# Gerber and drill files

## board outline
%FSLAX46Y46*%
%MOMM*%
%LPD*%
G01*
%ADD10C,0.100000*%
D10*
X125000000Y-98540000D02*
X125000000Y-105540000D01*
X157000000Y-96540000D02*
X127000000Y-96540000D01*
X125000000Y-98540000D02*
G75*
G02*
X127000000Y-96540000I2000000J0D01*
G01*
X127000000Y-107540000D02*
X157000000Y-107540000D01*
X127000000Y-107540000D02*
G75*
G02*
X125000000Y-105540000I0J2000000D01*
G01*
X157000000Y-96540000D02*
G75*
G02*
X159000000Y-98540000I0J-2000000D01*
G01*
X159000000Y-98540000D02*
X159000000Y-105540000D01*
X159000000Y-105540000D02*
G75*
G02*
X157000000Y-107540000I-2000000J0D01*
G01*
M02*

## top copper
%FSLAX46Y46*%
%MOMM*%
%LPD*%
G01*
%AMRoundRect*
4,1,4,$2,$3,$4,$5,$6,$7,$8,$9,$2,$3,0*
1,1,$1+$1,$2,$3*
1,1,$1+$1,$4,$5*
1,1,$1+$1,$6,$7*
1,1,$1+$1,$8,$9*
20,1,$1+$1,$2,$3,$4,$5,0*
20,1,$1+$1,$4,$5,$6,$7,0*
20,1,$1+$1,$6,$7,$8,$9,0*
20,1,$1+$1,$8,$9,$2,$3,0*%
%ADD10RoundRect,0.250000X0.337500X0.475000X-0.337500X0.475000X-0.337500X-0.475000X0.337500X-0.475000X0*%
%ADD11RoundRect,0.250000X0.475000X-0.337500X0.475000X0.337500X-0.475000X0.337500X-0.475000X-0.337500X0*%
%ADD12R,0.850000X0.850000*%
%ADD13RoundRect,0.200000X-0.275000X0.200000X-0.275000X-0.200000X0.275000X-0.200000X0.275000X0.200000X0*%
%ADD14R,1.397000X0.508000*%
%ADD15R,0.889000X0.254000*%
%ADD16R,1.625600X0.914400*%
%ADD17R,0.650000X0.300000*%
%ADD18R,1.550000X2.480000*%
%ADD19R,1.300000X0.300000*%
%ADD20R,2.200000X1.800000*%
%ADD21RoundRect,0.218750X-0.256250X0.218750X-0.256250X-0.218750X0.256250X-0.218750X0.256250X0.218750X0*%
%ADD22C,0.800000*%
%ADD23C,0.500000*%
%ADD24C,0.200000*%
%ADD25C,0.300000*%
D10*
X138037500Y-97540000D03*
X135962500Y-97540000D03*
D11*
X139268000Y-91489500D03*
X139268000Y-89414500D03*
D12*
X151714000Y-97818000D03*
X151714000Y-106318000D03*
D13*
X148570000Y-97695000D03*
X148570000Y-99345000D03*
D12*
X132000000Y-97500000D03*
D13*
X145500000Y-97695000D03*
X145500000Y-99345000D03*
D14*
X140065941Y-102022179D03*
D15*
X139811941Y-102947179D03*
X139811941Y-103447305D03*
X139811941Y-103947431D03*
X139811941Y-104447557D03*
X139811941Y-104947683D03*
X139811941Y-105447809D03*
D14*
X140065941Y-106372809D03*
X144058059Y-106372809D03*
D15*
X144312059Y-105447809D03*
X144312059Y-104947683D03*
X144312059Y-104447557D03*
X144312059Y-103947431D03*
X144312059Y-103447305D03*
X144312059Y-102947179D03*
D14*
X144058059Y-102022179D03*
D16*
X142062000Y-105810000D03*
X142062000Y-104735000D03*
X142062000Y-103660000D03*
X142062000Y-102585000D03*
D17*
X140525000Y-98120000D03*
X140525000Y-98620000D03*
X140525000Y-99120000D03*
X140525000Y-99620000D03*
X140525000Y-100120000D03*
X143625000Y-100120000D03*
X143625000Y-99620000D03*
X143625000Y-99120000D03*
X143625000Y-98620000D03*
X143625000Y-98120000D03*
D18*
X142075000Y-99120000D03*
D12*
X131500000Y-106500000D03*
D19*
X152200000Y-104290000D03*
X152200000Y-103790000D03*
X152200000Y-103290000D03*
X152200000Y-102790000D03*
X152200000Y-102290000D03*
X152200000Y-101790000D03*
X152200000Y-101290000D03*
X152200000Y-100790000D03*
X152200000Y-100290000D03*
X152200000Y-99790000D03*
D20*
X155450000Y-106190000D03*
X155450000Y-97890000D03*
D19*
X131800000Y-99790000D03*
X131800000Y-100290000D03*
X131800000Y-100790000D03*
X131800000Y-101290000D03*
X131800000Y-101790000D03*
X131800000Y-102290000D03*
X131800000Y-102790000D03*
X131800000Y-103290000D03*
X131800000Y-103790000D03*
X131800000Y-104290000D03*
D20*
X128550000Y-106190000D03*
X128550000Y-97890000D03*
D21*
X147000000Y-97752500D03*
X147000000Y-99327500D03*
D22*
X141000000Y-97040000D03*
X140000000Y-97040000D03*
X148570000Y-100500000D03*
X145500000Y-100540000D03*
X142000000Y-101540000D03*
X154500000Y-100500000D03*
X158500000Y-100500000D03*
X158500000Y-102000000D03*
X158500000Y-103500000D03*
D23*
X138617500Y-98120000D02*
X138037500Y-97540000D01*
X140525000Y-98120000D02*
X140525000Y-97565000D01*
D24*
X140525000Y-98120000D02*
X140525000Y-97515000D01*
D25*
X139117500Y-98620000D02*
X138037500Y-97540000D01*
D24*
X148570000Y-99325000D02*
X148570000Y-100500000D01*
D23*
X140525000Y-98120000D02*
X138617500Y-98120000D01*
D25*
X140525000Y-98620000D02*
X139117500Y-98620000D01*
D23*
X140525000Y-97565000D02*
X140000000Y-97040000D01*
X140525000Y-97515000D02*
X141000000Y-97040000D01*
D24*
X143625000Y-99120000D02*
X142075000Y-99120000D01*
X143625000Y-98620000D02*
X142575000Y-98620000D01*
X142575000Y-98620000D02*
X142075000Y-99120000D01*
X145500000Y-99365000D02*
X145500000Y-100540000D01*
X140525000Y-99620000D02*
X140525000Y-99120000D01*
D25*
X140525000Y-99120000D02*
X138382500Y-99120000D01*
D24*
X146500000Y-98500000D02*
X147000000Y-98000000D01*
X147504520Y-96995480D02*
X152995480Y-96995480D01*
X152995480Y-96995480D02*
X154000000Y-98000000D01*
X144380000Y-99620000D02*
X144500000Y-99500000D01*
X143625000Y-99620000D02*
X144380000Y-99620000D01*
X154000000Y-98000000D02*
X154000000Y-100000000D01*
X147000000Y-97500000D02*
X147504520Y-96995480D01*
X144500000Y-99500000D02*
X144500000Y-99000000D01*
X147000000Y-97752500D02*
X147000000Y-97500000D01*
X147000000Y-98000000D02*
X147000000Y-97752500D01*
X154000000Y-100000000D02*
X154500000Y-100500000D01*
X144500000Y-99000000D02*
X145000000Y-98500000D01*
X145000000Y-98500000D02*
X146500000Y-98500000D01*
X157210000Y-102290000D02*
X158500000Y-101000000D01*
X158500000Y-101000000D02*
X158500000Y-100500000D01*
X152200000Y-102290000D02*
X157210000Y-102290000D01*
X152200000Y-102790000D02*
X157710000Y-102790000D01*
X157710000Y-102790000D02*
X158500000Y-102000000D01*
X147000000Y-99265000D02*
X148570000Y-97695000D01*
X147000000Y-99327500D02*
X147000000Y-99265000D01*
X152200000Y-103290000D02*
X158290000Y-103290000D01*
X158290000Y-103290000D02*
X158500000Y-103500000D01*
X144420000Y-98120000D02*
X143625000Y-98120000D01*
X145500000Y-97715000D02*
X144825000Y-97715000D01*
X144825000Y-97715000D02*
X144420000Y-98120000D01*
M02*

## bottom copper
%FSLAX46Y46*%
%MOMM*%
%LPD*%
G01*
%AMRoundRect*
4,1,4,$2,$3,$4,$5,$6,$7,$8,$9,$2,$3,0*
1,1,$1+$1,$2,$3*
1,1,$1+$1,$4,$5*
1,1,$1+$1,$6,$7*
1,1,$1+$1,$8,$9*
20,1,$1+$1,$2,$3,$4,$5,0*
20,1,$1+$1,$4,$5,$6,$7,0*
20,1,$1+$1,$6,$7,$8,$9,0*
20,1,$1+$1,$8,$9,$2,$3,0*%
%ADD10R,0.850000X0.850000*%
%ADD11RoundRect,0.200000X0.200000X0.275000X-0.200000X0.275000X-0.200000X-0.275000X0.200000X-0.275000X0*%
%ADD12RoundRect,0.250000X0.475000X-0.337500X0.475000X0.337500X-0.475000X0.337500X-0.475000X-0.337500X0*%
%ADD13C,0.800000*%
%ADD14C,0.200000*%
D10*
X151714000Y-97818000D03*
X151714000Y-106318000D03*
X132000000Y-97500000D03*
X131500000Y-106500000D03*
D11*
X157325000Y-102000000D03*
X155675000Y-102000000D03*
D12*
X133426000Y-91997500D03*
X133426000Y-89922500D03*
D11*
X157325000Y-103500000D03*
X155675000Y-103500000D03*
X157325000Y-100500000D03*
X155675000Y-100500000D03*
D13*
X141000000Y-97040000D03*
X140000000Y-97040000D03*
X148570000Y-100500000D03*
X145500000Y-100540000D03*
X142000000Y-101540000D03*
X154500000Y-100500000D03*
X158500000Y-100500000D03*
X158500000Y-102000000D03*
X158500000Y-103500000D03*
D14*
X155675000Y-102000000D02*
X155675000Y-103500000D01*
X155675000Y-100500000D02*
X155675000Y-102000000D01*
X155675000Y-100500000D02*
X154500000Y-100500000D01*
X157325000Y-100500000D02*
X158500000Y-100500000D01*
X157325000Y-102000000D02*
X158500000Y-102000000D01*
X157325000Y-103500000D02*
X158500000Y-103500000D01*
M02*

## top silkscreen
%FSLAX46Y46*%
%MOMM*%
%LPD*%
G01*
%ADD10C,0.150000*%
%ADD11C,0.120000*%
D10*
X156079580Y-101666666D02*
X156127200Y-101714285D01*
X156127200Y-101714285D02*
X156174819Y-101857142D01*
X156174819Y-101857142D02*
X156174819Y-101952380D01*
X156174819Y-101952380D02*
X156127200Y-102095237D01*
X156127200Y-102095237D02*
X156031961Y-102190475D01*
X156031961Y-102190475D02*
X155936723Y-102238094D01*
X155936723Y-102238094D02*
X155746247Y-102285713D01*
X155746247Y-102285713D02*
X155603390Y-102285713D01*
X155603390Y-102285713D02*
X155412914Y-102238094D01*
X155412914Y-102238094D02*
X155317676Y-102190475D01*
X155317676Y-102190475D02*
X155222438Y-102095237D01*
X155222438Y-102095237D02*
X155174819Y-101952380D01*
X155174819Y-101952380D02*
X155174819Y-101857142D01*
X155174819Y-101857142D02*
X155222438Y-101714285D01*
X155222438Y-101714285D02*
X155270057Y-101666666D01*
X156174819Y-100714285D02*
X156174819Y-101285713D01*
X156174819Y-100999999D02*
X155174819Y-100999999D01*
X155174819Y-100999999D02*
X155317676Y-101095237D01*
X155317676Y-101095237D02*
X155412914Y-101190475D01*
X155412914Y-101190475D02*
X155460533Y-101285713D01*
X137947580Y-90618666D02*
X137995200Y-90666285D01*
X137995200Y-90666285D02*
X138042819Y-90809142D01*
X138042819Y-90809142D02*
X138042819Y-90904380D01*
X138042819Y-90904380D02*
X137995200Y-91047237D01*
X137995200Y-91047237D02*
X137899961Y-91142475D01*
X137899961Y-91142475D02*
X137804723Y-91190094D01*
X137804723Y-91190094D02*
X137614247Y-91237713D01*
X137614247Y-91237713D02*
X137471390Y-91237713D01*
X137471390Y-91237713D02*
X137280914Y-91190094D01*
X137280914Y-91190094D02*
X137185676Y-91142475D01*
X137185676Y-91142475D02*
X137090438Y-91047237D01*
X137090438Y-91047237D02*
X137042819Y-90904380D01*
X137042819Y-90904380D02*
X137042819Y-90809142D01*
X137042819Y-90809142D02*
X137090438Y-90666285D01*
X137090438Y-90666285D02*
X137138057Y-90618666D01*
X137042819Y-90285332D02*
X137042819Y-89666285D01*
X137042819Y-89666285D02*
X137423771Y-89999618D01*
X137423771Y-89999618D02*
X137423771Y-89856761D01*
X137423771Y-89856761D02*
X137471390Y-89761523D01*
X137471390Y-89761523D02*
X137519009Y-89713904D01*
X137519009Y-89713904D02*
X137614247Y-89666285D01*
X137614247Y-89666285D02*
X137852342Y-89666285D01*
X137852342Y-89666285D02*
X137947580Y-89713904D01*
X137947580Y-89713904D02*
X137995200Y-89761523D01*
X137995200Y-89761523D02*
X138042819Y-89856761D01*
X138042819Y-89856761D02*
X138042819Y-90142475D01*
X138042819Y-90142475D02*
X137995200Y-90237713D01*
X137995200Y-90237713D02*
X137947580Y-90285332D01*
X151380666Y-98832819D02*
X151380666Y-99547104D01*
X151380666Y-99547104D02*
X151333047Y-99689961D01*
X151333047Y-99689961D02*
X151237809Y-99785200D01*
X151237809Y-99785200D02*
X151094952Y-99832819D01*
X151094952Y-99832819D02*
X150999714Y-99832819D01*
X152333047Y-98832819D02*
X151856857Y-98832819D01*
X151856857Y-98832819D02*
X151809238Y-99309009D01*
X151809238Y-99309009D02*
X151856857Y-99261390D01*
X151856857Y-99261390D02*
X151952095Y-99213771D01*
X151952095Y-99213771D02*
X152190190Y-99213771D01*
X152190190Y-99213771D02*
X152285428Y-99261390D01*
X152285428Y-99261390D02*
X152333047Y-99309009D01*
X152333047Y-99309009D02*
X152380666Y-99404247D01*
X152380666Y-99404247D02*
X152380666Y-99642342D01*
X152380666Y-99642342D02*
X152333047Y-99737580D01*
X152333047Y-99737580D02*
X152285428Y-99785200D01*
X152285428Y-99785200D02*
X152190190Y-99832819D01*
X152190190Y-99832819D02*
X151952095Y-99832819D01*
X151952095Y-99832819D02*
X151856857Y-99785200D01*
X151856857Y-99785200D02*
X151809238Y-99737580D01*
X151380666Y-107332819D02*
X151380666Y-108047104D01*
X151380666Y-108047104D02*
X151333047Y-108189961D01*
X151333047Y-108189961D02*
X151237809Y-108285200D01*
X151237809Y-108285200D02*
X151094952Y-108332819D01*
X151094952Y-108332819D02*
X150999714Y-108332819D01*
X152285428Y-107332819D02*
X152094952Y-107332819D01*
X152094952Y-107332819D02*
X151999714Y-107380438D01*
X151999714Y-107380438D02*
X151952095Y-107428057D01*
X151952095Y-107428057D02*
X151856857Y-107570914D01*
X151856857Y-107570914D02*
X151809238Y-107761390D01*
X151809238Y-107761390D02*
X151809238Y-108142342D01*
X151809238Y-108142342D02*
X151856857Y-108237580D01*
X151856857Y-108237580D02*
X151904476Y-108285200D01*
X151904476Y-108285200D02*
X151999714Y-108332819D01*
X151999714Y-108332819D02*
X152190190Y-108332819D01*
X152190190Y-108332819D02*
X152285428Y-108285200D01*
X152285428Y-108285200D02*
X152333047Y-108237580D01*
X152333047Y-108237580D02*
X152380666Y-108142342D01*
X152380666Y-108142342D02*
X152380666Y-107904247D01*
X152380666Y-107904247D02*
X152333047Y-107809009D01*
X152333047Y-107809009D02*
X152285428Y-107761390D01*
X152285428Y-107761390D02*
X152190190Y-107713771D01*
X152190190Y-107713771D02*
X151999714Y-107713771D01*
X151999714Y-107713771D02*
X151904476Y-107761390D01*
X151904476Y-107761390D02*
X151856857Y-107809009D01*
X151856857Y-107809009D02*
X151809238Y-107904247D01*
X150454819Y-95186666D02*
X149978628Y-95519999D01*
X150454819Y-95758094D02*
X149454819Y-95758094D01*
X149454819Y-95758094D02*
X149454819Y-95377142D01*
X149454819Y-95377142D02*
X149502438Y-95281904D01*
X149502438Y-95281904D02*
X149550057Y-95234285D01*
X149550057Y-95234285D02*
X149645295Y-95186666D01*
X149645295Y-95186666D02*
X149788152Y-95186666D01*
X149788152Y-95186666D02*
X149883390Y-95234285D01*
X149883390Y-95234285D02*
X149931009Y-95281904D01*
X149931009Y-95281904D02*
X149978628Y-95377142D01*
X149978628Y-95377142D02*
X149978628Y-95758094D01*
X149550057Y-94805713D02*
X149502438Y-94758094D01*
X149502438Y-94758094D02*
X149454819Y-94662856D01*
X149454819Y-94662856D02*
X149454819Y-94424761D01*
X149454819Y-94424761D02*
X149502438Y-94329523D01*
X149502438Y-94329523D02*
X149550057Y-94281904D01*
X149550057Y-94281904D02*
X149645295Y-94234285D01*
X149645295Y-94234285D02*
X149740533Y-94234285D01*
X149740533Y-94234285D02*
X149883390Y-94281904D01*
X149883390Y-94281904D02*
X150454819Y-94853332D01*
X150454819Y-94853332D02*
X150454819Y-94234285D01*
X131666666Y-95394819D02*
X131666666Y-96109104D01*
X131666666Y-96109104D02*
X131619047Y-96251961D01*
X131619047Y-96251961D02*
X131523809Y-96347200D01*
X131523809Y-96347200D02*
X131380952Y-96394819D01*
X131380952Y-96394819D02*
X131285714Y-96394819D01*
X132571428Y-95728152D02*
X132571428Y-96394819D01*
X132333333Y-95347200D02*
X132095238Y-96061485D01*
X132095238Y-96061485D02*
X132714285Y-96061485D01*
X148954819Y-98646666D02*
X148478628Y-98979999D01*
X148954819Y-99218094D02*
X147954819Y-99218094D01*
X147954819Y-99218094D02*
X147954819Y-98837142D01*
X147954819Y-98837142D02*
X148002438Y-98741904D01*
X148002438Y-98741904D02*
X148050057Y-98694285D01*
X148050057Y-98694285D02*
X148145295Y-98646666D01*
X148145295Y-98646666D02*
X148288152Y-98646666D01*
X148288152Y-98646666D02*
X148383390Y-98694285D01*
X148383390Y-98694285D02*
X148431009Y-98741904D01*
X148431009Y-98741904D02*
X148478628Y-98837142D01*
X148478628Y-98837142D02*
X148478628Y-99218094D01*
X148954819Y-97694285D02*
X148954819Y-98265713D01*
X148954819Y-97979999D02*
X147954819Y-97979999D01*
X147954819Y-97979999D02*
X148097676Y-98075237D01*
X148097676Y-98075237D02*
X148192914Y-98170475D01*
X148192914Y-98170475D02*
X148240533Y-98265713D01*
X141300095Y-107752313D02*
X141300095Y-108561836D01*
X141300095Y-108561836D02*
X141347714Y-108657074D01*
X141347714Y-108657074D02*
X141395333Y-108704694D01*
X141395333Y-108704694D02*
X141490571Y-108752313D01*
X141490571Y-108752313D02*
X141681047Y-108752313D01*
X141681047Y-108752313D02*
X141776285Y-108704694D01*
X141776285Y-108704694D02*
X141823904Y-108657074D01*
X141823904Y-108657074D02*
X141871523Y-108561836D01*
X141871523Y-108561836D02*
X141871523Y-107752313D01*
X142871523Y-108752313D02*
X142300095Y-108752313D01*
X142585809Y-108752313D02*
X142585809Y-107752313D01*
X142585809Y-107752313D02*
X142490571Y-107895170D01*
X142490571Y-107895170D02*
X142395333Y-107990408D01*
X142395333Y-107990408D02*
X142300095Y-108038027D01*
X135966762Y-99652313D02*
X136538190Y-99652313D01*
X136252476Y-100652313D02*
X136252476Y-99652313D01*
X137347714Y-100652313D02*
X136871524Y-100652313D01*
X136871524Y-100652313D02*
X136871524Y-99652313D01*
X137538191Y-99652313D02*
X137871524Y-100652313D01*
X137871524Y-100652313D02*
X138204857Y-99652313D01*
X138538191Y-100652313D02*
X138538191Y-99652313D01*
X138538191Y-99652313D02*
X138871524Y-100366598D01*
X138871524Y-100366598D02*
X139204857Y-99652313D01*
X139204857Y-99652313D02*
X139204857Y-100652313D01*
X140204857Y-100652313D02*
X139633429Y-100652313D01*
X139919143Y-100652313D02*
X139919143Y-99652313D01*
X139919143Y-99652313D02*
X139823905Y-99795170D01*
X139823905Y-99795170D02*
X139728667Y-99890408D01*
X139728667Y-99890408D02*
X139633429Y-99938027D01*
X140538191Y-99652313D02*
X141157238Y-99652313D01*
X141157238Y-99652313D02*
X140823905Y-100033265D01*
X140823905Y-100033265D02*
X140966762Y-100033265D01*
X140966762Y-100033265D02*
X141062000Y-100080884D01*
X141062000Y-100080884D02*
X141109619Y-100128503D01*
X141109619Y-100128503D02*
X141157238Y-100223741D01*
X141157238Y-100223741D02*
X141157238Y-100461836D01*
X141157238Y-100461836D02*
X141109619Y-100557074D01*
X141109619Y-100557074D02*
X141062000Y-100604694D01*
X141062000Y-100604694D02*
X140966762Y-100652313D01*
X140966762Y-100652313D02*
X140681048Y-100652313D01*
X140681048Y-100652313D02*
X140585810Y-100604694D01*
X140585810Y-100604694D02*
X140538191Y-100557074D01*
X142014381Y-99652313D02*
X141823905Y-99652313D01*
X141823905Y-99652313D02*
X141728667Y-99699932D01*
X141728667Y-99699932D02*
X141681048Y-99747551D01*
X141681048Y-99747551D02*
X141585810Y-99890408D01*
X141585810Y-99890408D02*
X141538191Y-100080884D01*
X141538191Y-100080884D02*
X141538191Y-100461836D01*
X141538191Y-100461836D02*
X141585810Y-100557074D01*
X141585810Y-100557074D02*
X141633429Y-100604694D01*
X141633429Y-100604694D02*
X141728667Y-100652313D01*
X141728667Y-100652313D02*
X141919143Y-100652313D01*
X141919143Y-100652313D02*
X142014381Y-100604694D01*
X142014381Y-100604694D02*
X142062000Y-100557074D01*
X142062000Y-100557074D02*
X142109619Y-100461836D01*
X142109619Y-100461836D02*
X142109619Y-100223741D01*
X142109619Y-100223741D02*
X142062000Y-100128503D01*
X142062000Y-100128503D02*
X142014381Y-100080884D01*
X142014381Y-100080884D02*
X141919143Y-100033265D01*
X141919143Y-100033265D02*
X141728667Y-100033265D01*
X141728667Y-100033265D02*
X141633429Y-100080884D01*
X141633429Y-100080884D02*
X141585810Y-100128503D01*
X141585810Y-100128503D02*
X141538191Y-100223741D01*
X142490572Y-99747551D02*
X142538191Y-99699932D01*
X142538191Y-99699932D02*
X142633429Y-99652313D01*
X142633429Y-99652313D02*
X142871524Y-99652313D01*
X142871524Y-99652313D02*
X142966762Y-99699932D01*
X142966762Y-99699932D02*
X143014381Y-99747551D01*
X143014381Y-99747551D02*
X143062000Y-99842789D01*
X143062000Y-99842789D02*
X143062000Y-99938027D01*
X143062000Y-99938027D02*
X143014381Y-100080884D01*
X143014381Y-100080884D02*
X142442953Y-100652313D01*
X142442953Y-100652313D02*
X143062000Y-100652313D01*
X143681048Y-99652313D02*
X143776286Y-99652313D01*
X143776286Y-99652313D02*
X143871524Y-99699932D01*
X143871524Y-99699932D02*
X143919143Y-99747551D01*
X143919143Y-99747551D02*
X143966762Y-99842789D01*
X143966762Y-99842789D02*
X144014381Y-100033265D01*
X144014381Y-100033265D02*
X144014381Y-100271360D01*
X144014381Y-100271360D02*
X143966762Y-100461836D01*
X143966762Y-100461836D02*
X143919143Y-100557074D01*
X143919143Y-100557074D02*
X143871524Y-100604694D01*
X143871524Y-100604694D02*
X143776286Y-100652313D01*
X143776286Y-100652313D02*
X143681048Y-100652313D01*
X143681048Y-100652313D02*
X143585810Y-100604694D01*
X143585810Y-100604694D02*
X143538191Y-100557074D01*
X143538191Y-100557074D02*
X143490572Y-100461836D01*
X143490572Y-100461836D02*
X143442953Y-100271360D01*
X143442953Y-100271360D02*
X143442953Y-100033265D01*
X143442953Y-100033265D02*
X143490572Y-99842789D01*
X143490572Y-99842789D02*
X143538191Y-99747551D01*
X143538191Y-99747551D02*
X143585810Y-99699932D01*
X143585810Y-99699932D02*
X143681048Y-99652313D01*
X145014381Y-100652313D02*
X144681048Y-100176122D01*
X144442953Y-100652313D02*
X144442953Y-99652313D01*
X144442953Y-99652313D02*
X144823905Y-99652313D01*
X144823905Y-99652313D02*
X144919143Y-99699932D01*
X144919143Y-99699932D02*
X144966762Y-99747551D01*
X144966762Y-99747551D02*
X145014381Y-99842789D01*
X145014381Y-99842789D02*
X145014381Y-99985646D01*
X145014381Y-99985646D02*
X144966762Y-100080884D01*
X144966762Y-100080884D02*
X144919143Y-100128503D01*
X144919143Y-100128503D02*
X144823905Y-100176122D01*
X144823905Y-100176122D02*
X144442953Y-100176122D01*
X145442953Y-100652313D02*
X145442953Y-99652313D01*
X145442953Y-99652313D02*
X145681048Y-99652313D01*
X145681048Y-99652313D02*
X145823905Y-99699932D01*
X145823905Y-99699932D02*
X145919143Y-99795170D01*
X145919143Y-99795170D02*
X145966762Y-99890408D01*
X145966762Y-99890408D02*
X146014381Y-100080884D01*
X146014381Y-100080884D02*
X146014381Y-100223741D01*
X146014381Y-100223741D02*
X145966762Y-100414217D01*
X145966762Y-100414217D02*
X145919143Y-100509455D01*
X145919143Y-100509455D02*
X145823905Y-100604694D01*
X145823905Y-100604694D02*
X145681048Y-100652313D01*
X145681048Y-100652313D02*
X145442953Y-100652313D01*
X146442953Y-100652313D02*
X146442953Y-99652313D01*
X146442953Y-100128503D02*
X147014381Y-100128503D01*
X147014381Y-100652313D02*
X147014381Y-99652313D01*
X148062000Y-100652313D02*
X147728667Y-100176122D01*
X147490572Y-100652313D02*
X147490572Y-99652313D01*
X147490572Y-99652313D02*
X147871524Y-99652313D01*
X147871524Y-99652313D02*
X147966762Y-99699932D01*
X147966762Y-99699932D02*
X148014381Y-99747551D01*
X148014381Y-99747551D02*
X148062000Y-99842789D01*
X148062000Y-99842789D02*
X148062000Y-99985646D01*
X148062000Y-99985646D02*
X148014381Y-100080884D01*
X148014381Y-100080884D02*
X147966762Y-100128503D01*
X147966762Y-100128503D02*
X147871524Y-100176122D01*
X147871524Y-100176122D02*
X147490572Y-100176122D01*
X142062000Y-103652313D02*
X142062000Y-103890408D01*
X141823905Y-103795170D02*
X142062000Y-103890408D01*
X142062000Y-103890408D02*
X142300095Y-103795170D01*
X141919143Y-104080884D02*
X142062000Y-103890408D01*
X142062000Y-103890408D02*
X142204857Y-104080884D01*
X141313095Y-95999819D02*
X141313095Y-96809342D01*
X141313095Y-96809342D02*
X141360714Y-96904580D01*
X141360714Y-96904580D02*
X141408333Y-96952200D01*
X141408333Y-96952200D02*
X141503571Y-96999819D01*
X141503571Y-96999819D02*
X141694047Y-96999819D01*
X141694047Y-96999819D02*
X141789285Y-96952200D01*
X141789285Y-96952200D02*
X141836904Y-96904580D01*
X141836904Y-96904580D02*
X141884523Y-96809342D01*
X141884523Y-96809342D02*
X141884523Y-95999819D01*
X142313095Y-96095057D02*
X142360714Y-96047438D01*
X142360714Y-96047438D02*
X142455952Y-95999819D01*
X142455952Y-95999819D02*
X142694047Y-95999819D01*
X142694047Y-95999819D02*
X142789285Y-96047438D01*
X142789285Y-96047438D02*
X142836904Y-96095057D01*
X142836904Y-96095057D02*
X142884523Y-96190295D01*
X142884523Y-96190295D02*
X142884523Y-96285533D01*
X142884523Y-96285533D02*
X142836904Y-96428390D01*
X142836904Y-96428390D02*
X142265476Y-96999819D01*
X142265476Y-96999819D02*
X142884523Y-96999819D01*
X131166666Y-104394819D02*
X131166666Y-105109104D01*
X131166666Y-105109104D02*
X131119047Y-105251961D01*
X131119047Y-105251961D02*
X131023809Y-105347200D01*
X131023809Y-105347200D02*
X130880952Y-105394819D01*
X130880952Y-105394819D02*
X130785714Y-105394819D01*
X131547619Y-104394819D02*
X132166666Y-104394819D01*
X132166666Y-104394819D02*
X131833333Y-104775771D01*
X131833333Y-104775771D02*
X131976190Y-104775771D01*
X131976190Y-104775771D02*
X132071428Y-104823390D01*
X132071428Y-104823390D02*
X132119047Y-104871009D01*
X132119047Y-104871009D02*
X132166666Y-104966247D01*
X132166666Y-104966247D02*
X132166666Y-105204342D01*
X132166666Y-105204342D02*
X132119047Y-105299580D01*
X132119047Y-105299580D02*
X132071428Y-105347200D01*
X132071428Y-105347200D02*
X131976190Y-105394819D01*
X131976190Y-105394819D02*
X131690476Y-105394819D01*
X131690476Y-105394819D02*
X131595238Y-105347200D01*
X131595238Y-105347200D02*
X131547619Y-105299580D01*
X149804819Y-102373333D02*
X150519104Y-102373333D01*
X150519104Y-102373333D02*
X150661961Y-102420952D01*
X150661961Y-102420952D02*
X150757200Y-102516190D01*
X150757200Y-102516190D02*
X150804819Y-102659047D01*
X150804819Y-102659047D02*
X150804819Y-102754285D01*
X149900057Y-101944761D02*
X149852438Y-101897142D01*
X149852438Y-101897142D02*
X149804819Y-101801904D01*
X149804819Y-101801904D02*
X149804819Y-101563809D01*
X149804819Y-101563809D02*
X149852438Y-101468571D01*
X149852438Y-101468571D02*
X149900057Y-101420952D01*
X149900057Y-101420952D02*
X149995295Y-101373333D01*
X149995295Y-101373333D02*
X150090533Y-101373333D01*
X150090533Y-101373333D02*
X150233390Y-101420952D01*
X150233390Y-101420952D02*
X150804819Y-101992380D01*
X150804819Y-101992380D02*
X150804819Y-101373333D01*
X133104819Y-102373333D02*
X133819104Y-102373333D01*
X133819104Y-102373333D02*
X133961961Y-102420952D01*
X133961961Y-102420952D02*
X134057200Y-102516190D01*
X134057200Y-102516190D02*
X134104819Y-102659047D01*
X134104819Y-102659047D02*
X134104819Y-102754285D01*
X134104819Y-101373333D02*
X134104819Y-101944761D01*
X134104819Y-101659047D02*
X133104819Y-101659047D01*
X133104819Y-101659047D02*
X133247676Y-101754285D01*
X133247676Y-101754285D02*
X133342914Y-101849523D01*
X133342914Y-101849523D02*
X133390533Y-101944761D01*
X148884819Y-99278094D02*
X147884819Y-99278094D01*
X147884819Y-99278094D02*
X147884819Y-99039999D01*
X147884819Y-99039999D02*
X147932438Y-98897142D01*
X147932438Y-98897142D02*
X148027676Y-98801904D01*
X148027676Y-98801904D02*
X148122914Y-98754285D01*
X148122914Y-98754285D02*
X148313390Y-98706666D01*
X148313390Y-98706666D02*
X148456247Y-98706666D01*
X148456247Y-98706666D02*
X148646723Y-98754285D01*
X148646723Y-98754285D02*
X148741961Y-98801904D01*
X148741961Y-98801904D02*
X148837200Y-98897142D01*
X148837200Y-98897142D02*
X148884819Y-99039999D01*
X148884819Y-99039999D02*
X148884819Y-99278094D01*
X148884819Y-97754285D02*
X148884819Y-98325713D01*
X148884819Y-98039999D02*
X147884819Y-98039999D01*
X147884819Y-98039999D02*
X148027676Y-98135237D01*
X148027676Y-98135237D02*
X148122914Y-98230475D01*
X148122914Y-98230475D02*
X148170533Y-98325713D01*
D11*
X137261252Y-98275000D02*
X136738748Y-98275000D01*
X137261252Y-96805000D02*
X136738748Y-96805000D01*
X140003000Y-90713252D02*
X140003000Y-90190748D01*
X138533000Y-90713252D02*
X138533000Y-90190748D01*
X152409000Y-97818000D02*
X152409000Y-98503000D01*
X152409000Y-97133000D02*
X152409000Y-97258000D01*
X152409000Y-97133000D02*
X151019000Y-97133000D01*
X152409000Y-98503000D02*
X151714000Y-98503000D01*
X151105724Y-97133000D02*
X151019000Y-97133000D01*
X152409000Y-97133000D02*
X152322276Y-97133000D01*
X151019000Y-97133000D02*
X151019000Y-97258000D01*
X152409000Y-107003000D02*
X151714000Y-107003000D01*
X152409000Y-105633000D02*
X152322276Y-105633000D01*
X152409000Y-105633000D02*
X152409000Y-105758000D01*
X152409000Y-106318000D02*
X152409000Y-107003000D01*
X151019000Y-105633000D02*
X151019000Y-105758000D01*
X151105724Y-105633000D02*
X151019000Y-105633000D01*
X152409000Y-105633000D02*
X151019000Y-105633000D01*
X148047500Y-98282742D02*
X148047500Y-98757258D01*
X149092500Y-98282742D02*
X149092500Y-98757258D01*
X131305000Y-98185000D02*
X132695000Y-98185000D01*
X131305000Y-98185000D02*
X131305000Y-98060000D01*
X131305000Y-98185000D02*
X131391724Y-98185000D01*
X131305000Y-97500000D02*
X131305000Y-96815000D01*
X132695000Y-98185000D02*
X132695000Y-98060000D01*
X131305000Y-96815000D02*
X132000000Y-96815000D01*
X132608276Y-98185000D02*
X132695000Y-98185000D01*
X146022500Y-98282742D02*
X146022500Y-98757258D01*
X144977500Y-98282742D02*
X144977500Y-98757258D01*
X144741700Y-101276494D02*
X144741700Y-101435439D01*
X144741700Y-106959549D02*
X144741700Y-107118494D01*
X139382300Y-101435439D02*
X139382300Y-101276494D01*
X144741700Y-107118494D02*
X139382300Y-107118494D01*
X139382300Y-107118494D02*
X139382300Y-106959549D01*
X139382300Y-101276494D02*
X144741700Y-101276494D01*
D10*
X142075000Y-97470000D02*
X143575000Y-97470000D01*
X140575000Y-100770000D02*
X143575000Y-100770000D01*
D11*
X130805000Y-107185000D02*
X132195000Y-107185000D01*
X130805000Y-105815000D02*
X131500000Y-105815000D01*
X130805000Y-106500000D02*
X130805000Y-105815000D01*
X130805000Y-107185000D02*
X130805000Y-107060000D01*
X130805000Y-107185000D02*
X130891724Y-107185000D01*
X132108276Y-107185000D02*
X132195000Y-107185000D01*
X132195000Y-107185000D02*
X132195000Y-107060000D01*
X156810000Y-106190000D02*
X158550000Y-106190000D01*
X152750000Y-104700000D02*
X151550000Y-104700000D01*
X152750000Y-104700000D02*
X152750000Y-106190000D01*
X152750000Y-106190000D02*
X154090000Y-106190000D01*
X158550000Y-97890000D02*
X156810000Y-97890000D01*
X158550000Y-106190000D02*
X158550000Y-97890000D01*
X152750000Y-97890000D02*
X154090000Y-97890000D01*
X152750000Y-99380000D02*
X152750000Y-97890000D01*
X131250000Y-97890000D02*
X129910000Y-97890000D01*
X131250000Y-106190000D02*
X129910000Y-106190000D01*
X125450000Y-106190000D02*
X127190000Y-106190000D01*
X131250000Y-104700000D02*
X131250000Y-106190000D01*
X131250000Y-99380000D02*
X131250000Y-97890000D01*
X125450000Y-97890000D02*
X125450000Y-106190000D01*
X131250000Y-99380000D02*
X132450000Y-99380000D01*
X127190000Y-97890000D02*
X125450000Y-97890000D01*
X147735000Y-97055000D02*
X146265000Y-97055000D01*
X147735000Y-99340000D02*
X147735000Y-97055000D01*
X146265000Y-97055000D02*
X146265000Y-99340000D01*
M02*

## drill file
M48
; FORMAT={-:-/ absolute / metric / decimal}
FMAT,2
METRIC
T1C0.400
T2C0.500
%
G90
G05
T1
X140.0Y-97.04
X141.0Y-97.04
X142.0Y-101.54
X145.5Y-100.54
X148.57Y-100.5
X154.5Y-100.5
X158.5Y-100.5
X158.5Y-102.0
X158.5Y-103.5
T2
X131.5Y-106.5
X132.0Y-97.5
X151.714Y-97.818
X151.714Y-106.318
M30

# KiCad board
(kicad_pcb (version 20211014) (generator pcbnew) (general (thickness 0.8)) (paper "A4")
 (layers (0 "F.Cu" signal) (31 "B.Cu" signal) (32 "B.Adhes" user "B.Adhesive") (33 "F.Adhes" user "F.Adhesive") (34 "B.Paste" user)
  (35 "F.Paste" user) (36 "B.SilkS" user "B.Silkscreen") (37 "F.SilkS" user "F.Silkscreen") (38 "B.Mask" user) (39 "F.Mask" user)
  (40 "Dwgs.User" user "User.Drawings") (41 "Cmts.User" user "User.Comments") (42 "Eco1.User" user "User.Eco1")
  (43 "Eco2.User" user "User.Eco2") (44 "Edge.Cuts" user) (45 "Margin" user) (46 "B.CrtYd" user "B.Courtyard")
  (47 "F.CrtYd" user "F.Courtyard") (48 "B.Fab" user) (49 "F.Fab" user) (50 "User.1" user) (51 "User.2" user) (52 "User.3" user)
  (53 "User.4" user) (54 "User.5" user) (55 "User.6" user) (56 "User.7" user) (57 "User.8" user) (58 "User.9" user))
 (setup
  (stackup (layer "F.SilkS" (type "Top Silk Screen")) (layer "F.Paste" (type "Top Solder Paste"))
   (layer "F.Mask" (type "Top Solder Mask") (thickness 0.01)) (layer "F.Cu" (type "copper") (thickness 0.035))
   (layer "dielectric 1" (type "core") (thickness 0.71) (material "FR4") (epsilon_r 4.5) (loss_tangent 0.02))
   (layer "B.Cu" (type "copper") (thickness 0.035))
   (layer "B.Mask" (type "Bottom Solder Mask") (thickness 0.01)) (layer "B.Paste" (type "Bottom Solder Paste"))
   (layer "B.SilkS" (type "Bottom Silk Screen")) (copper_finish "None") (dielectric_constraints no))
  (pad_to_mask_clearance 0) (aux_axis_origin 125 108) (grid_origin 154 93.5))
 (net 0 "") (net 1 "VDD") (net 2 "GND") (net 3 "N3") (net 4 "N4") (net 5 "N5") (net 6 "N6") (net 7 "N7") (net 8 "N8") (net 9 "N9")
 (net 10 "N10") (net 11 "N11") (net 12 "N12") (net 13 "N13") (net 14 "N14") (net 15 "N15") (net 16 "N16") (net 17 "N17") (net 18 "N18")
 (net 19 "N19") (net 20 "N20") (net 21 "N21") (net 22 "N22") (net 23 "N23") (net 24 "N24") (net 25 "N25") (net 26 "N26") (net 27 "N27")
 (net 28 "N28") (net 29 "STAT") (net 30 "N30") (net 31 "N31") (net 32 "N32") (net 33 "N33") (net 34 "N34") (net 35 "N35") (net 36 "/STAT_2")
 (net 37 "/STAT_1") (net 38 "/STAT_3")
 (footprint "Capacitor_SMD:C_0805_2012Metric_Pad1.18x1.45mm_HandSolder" (layer "F.Cu") (at 137 97.54 180)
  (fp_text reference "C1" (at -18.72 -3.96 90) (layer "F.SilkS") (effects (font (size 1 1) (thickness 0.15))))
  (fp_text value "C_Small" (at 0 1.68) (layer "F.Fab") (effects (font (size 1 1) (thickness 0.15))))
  (fp_line (start -0.261252 -0.735) (end 0.261252 -0.735) (layer "F.SilkS") (width 0.12))
  (fp_line (start -0.261252 0.735) (end 0.261252 0.735) (layer "F.SilkS") (width 0.12))
  (pad "1" smd roundrect (at -1.0375 0 180) (size 1.175 1.45) (layers "F.Cu" "F.Paste" "F.Mask") (roundrect_rratio 0.212766) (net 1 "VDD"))
  (pad "2" smd roundrect (at 1.0375 0 180) (size 1.175 1.45) (layers "F.Cu" "F.Paste" "F.Mask") (roundrect_rratio 0.212766) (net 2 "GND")))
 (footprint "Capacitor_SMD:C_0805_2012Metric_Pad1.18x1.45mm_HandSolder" (layer "F.Cu") (at 139.268 90.452 90)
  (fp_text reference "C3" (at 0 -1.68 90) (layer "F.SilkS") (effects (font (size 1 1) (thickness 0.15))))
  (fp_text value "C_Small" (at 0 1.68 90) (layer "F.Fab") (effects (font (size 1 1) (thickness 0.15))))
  (fp_line (start -0.261252 0.735) (end 0.261252 0.735) (layer "F.SilkS") (width 0.12))
  (fp_line (start -0.261252 -0.735) (end 0.261252 -0.735) (layer "F.SilkS") (width 0.12))
  (pad "1" smd roundrect (at -1.0375 0 90) (size 1.175 1.45) (layers "F.Cu" "F.Paste" "F.Mask") (roundrect_rratio 0.212766) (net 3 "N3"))
  (pad "2" smd roundrect (at 1.0375 0 90) (size 1.175 1.45) (layers "F.Cu" "F.Paste" "F.Mask") (roundrect_rratio 0.212766) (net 2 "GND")))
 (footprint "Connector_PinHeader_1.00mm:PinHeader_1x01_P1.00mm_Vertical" (layer "F.Cu") (at 151.714 97.818 180)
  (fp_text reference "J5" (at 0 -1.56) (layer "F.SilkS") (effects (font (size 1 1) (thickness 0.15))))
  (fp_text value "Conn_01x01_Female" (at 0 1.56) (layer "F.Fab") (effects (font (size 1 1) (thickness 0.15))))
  (fp_line (start -0.695 0) (end -0.695 -0.685) (layer "F.SilkS") (width 0.12))
  (fp_line (start -0.695 0.685) (end -0.695 0.56) (layer "F.SilkS") (width 0.12))
  (fp_line (start -0.695 0.685) (end 0.695 0.685) (layer "F.SilkS") (width 0.12))
  (fp_line (start -0.695 -0.685) (end 0 -0.685) (layer "F.SilkS") (width 0.12))
  (fp_line (start 0.608276 0.685) (end 0.695 0.685) (layer "F.SilkS") (width 0.12))
  (fp_line (start -0.695 0.685) (end -0.608276 0.685) (layer "F.SilkS") (width 0.12))
  (fp_line (start 0.695 0.685) (end 0.695 0.56) (layer "F.SilkS") (width 0.12))
  (pad "1" thru_hole rect (at 0 0 180) (size 0.85 0.85) (drill 0.5) (layers *.Cu *.Mask) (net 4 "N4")))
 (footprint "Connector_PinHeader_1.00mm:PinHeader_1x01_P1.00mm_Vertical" (layer "F.Cu") (at 151.714 106.318 180)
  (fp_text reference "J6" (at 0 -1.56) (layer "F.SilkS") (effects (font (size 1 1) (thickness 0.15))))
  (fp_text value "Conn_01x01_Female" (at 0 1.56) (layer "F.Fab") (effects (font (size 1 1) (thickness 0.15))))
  (fp_line (start -0.695 -0.685) (end 0 -0.685) (layer "F.SilkS") (width 0.12))
  (fp_line (start -0.695 0.685) (end -0.608276 0.685) (layer "F.SilkS") (width 0.12))
  (fp_line (start -0.695 0.685) (end -0.695 0.56) (layer "F.SilkS") (width 0.12))
  (fp_line (start -0.695 0) (end -0.695 -0.685) (layer "F.SilkS") (width 0.12))
  (fp_line (start 0.695 0.685) (end 0.695 0.56) (layer "F.SilkS") (width 0.12))
  (fp_line (start 0.608276 0.685) (end 0.695 0.685) (layer "F.SilkS") (width 0.12))
  (fp_line (start -0.695 0.685) (end 0.695 0.685) (layer "F.SilkS") (width 0.12))
  (pad "1" thru_hole rect (at 0 0 180) (size 0.85 0.85) (drill 0.5) (layers *.Cu *.Mask) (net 2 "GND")))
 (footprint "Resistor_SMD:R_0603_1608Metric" (layer "F.Cu") (at 148.57 98.52 -90)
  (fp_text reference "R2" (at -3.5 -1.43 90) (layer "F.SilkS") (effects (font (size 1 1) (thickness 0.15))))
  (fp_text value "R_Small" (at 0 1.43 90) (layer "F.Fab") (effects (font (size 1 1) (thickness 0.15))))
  (fp_line (start -0.237258 0.5225) (end 0.237258 0.5225) (layer "F.SilkS") (width 0.12))
  (fp_line (start -0.237258 -0.5225) (end 0.237258 -0.5225) (layer "F.SilkS") (width 0.12))
  (pad "1" smd roundrect (at -0.825 0 270) (size 0.8 0.95) (layers "F.Cu" "F.Paste" "F.Mask") (roundrect_rratio 0.25) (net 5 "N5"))
  (pad "2" smd roundrect (at 0.825 0 270) (size 0.8 0.95) (layers "F.Cu" "F.Paste" "F.Mask") (roundrect_rratio 0.25) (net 1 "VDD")))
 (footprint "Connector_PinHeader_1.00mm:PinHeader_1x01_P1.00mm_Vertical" (layer "F.Cu") (at 132 97.5)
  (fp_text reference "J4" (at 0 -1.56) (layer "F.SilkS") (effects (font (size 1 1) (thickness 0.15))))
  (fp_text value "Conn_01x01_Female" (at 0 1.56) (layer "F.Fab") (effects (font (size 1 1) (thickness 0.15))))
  (fp_line (start -0.695 0.685) (end 0.695 0.685) (layer "F.SilkS") (width 0.12))
  (fp_line (start -0.695 0.685) (end -0.695 0.56) (layer "F.SilkS") (width 0.12))
  (fp_line (start -0.695 0.685) (end -0.608276 0.685) (layer "F.SilkS") (width 0.12))
  (fp_line (start -0.695 0) (end -0.695 -0.685) (layer "F.SilkS") (width 0.12))
  (fp_line (start 0.695 0.685) (end 0.695 0.56) (layer "F.SilkS") (width 0.12))
  (fp_line (start -0.695 -0.685) (end 0 -0.685) (layer "F.SilkS") (width 0.12))
  (fp_line (start 0.608276 0.685) (end 0.695 0.685) (layer "F.SilkS") (width 0.12))
  (pad "1" thru_hole rect (at 0 0) (size 0.85 0.85) (drill 0.5) (layers *.Cu *.Mask) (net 4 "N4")))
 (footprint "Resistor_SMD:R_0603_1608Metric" (layer "F.Cu") (at 145.5 98.52 -90)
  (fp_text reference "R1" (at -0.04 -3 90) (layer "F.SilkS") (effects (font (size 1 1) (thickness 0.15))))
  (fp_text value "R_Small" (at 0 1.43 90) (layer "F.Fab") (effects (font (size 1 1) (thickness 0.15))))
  (fp_line (start -0.237258 -0.5225) (end 0.237258 -0.5225) (layer "F.SilkS") (width 0.12))
  (fp_line (start -0.237258 0.5225) (end 0.237258 0.5225) (layer "F.SilkS") (width 0.12))
  (pad "1" smd roundrect (at -0.825 0 270) (size 0.8 0.95) (layers "F.Cu" "F.Paste" "F.Mask") (roundrect_rratio 0.25) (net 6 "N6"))
  (pad "2" smd roundrect (at 0.825 0 270) (size 0.8 0.95) (layers "F.Cu" "F.Paste" "F.Mask") (roundrect_rratio 0.25) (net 2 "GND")))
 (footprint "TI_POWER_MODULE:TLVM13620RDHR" (layer "F.Cu") (at 142.062 104.197494)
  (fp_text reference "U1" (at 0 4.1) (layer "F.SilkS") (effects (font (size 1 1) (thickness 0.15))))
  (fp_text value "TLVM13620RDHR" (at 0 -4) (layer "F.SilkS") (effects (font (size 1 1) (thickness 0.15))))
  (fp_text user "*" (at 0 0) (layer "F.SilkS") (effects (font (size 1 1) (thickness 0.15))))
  (fp_line (start 2.6797 -2.921) (end 2.6797 -2.762055) (layer "F.SilkS") (width 0.12))
  (fp_line (start 2.6797 2.762055) (end 2.6797 2.921) (layer "F.SilkS") (width 0.12))
  (fp_line (start -2.6797 -2.762055) (end -2.6797 -2.921) (layer "F.SilkS") (width 0.12))
  (fp_line (start 2.6797 2.921) (end -2.6797 2.921) (layer "F.SilkS") (width 0.12))
  (fp_line (start -2.6797 2.921) (end -2.6797 2.762055) (layer "F.SilkS") (width 0.12))
  (fp_line (start -2.6797 -2.921) (end 2.6797 -2.921) (layer "F.SilkS") (width 0.12))
  (pad "1" smd rect (at -1.996059 -2.175315) (size 1.397 0.508) (layers "F.Cu" "F.Paste" "F.Mask") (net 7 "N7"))
  (pad "2" smd rect (at -2.250059 -1.250315) (size 0.889 0.254) (layers "F.Cu" "F.Paste" "F.Mask") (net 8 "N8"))
  (pad "3" smd rect (at -2.250059 -0.750189) (size 0.889 0.254) (layers "F.Cu" "F.Paste" "F.Mask") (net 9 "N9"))
  (pad "4" smd rect (at -2.250059 -0.250063) (size 0.889 0.254) (layers "F.Cu" "F.Paste" "F.Mask") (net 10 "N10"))
  (pad "5" smd rect (at -2.250059 0.250063) (size 0.889 0.254) (layers "F.Cu" "F.Paste" "F.Mask") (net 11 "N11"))
  (pad "6" smd rect (at -2.250059 0.750189) (size 0.889 0.254) (layers "F.Cu" "F.Paste" "F.Mask") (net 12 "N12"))
  (pad "7" smd rect (at -2.250059 1.250315) (size 0.889 0.254) (layers "F.Cu" "F.Paste" "F.Mask") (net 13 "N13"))
  (pad "8" smd rect (at -1.996059 2.175315) (size 1.397 0.508) (layers "F.Cu" "F.Paste" "F.Mask") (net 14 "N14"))
  (pad "9" smd rect (at 1.996059 2.175315) (size 1.397 0.508) (layers "F.Cu" "F.Paste" "F.Mask") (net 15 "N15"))
  (pad "10" smd rect (at 2.250059 1.250315) (size 0.889 0.254) (layers "F.Cu" "F.Paste" "F.Mask") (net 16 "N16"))
  (pad "11" smd rect (at 2.250059 0.750189) (size 0.889 0.254) (layers "F.Cu" "F.Paste" "F.Mask") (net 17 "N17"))
  (pad "12" smd rect (at 2.250059 0.250063) (size 0.889 0.254) (layers "F.Cu" "F.Paste" "F.Mask") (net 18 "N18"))
  (pad "13" smd rect (at 2.250059 -0.250063) (size 0.889 0.254) (layers "F.Cu" "F.Paste" "F.Mask") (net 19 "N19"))
  (pad "14" smd rect (at 2.250059 -0.750189) (size 0.889 0.254) (layers "F.Cu" "F.Paste" "F.Mask") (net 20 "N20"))
  (pad "15" smd rect (at 2.250059 -1.250315) (size 0.889 0.254) (layers "F.Cu" "F.Paste" "F.Mask") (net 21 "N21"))
  (pad "16" smd rect (at 1.996059 -2.175315) (size 1.397 0.508) (layers "F.Cu" "F.Paste" "F.Mask") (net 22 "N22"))
  (pad "17" smd rect (at 0 1.612506) (size 1.6256 0.9144) (layers "F.Cu" "F.Mask") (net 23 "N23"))
  (pad "18" smd rect (at 0 0.537506) (size 1.6256 0.9144) (layers "F.Cu" "F.Mask") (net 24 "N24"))
  (pad "19" smd rect (at 0 -0.537494) (size 1.6256 0.9144) (layers "F.Cu" "F.Mask") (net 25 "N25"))
  (pad "20" smd rect (at 0 -1.612494) (size 1.6256 0.9144) (layers "F.Cu" "F.Mask") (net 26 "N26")))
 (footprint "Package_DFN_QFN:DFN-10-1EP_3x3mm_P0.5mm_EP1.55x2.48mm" (layer "F.Cu") (at 142.075 99.12)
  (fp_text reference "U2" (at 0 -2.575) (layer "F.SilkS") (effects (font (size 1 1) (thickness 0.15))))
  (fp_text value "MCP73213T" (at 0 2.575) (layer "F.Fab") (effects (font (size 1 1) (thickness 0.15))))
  (fp_line (start 0 -1.65) (end 1.5 -1.65) (layer "F.SilkS") (width 0.15))
  (fp_line (start -1.5 1.65) (end 1.5 1.65) (layer "F.SilkS") (width 0.15))
  (pad "" smd rect (at 0.3875 -0.62) (size 0.6 1.05) (layers "F.Paste"))
  (pad "" smd rect (at -0.3875 0.62) (size 0.6 1.05) (layers "F.Paste"))
  (pad "" smd rect (at 0.3875 0.62) (size 0.6 1.05) (layers "F.Paste"))
  (pad "" smd rect (at -0.3875 -0.62) (size 0.6 1.05) (layers "F.Paste"))
  (pad "1" smd rect (at -1.55 -1) (size 0.65 0.3) (layers "F.Cu" "F.Paste" "F.Mask") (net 1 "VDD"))
  (pad "2" smd rect (at -1.55 -0.5) (size 0.65 0.3) (layers "F.Cu" "F.Paste" "F.Mask") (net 1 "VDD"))
  (pad "3" smd rect (at -1.55 0) (size 0.65 0.3) (layers "F.Cu" "F.Paste" "F.Mask") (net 3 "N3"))
  (pad "4" smd rect (at -1.55 0.5) (size 0.65 0.3) (layers "F.Cu" "F.Paste" "F.Mask") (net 3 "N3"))
  (pad "5" smd rect (at -1.55 1) (size 0.65 0.3) (layers "F.Cu" "F.Paste" "F.Mask") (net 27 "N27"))
  (pad "6" smd rect (at 1.55 1) (size 0.65 0.3) (layers "F.Cu" "F.Paste" "F.Mask") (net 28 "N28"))
  (pad "7" smd rect (at 1.55 0.5) (size 0.65 0.3) (layers "F.Cu" "F.Paste" "F.Mask") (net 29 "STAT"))
  (pad "8" smd rect (at 1.55 0) (size 0.65 0.3) (layers "F.Cu" "F.Paste" "F.Mask") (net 2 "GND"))
  (pad "9" smd rect (at 1.55 -0.5) (size 0.65 0.3) (layers "F.Cu" "F.Paste" "F.Mask") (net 2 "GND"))
  (pad "10" smd rect (at 1.55 -1) (size 0.65 0.3) (layers "F.Cu" "F.Paste" "F.Mask") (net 6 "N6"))
  (pad "11" smd rect (at 0 0) (size 1.55 2.48) (layers "F.Cu" "F.Mask") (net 2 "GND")))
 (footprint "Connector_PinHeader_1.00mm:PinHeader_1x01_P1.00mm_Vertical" (layer "F.Cu") (at 131.5 106.5)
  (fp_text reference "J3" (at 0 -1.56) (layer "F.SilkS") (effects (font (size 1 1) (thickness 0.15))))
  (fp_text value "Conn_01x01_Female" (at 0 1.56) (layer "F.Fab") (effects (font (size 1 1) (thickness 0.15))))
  (fp_line (start -0.695 0.685) (end 0.695 0.685) (layer "F.SilkS") (width 0.12))
  (fp_line (start -0.695 -0.685) (end 0 -0.685) (layer "F.SilkS") (width 0.12))
  (fp_line (start -0.695 0) (end -0.695 -0.685) (layer "F.SilkS") (width 0.12))
  (fp_line (start -0.695 0.685) (end -0.695 0.56) (layer "F.SilkS") (width 0.12))
  (fp_line (start -0.695 0.685) (end -0.608276 0.685) (layer "F.SilkS") (width 0.12))
  (fp_line (start 0.608276 0.685) (end 0.695 0.685) (layer "F.SilkS") (width 0.12))
  (fp_line (start 0.695 0.685) (end 0.695 0.56) (layer "F.SilkS") (width 0.12))
  (pad "1" thru_hole rect (at 0 0) (size 0.85 0.85) (drill 0.5) (layers *.Cu *.Mask) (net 3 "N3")))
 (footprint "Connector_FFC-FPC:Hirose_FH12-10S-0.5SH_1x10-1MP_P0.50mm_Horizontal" (layer "F.Cu") (at 154.05 102.04 90)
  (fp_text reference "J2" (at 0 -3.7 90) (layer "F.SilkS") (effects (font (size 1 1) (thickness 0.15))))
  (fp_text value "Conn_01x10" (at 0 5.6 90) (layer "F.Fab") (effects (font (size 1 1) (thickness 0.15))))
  (fp_line (start -4.15 2.76) (end -4.15 4.5) (layer "F.SilkS") (width 0.12))
  (fp_line (start -2.66 -1.3) (end -2.66 -2.5) (layer "F.SilkS") (width 0.12))
  (fp_line (start -2.66 -1.3) (end -4.15 -1.3) (layer "F.SilkS") (width 0.12))
  (fp_line (start -4.15 -1.3) (end -4.15 0.04) (layer "F.SilkS") (width 0.12))
  (fp_line (start 4.15 4.5) (end 4.15 2.76) (layer "F.SilkS") (width 0.12))
  (fp_line (start -4.15 4.5) (end 4.15 4.5) (layer "F.SilkS") (width 0.12))
  (fp_line (start 4.15 -1.3) (end 4.15 0.04) (layer "F.SilkS") (width 0.12))
  (fp_line (start 2.66 -1.3) (end 4.15 -1.3) (layer "F.SilkS") (width 0.12))
  (pad "1" smd rect (at -2.25 -1.85 90) (size 0.3 1.3) (layers "F.Cu" "F.Paste" "F.Mask") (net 2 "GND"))
  (pad "2" smd rect (at -1.75 -1.85 90) (size 0.3 1.3) (layers "F.Cu" "F.Paste" "F.Mask") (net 2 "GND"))
  (pad "3" smd rect (at -1.25 -1.85 90) (size 0.3 1.3) (layers "F.Cu" "F.Paste" "F.Mask") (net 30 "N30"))
  (pad "4" smd rect (at -0.75 -1.85 90) (size 0.3 1.3) (layers "F.Cu" "F.Paste" "F.Mask") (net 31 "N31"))
  (pad "5" smd rect (at -0.25 -1.85 90) (size 0.3 1.3) (layers "F.Cu" "F.Paste" "F.Mask") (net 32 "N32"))
  (pad "6" smd rect (at 0.25 -1.85 90) (size 0.3 1.3) (layers "F.Cu" "F.Paste" "F.Mask") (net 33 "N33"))
  (pad "7" smd rect (at 0.75 -1.85 90) (size 0.3 1.3) (layers "F.Cu" "F.Paste" "F.Mask") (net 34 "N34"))
  (pad "8" smd rect (at 1.25 -1.85 90) (size 0.3 1.3) (layers "F.Cu" "F.Paste" "F.Mask") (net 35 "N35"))
  (pad "9" smd rect (at 1.75 -1.85 90) (size 0.3 1.3) (layers "F.Cu" "F.Paste" "F.Mask") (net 1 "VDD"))
  (pad "10" smd rect (at 2.25 -1.85 90) (size 0.3 1.3) (layers "F.Cu" "F.Paste" "F.Mask") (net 1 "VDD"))
  (pad "MP" smd rect (at -4.15 1.4 90) (size 1.8 2.2) (layers "F.Cu" "F.Paste" "F.Mask"))
  (pad "MP" smd rect (at 4.15 1.4 90) (size 1.8 2.2) (layers "F.Cu" "F.Paste" "F.Mask")))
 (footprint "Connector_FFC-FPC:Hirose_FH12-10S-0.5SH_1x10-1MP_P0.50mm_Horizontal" (layer "F.Cu") (at 129.95 102.04 -90)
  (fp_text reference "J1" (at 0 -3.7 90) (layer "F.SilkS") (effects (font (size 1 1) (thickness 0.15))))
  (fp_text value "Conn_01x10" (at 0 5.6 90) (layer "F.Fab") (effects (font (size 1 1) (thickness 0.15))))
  (fp_line (start -4.15 -1.3) (end -4.15 0.04) (layer "F.SilkS") (width 0.12))
  (fp_line (start 4.15 -1.3) (end 4.15 0.04) (layer "F.SilkS") (width 0.12))
  (fp_line (start 4.15 4.5) (end 4.15 2.76) (layer "F.SilkS") (width 0.12))
  (fp_line (start 2.66 -1.3) (end 4.15 -1.3) (layer "F.SilkS") (width 0.12))
  (fp_line (start -2.66 -1.3) (end -4.15 -1.3) (layer "F.SilkS") (width 0.12))
  (fp_line (start -4.15 4.5) (end 4.15 4.5) (layer "F.SilkS") (width 0.12))
  (fp_line (start -2.66 -1.3) (end -2.66 -2.5) (layer "F.SilkS") (width 0.12))
  (fp_line (start -4.15 2.76) (end -4.15 4.5) (layer "F.SilkS") (width 0.12))
  (pad "1" smd rect (at -2.25 -1.85 270) (size 0.3 1.3) (layers "F.Cu" "F.Paste" "F.Mask") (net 1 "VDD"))
  (pad "2" smd rect (at -1.75 -1.85 270) (size 0.3 1.3) (layers "F.Cu" "F.Paste" "F.Mask") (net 1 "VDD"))
  (pad "3" smd rect (at -1.25 -1.85 270) (size 0.3 1.3) (layers "F.Cu" "F.Paste" "F.Mask") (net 35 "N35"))
  (pad "4" smd rect (at -0.75 -1.85 270) (size 0.3 1.3) (layers "F.Cu" "F.Paste" "F.Mask") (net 34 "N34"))
  (pad "5" smd rect (at -0.25 -1.85 270) (size 0.3 1.3) (layers "F.Cu" "F.Paste" "F.Mask") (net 33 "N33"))
  (pad "6" smd rect (at 0.25 -1.85 270) (size 0.3 1.3) (layers "F.Cu" "F.Paste" "F.Mask") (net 32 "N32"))
  (pad "7" smd rect (at 0.75 -1.85 270) (size 0.3 1.3) (layers "F.Cu" "F.Paste" "F.Mask") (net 31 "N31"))
  (pad "8" smd rect (at 1.25 -1.85 270) (size 0.3 1.3) (layers "F.Cu" "F.Paste" "F.Mask") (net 30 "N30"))
  (pad "9" smd rect (at 1.75 -1.85 270) (size 0.3 1.3) (layers "F.Cu" "F.Paste" "F.Mask") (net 2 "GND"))
  (pad "10" smd rect (at 2.25 -1.85 270) (size 0.3 1.3) (layers "F.Cu" "F.Paste" "F.Mask") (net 2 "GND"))
  (pad "MP" smd rect (at 4.15 1.4 270) (size 1.8 2.2) (layers "F.Cu" "F.Paste" "F.Mask"))
  (pad "MP" smd rect (at -4.15 1.4 270) (size 1.8 2.2) (layers "F.Cu" "F.Paste" "F.Mask")))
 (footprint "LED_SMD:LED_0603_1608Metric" (layer "F.Cu") (at 147 98.54 -90)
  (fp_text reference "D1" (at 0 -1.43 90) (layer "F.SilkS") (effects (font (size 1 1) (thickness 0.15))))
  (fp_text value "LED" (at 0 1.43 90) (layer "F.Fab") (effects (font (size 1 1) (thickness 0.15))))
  (fp_line (start -1.485 -0.735) (end -1.485 0.735) (layer "F.SilkS") (width 0.12))
  (fp_line (start 0.8 -0.735) (end -1.485 -0.735) (layer "F.SilkS") (width 0.12))
  (fp_line (start -1.485 0.735) (end 0.8 0.735) (layer "F.SilkS") (width 0.12))
  (pad "1" smd roundrect (at -0.7875 0 270) (size 0.875 0.95) (layers "F.Cu" "F.Paste" "F.Mask") (roundrect_rratio 0.25) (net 29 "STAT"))
  (pad "2" smd roundrect (at 0.7875 0 270) (size 0.875 0.95) (layers "F.Cu" "F.Paste" "F.Mask") (roundrect_rratio 0.25) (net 5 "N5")))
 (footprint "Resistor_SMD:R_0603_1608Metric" (layer "B.Cu") (at 156.5 102 180)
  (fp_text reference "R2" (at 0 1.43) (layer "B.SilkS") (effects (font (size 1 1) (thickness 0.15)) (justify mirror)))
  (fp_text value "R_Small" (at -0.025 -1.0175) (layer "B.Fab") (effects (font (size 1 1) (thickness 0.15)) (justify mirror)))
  (pad "1" smd roundrect (at -0.825 0 180) (size 0.8 0.95) (layers "B.Cu" "B.Paste" "B.Mask") (roundrect_rratio 0.25) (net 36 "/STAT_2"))
  (pad "2" smd roundrect (at 0.825 0 180) (size 0.8 0.95) (layers "B.Cu" "B.Paste" "B.Mask") (roundrect_rratio 0.25) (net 29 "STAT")))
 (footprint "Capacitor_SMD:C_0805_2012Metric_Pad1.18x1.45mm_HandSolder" (layer "B.Cu") (at 133.426 90.96 90)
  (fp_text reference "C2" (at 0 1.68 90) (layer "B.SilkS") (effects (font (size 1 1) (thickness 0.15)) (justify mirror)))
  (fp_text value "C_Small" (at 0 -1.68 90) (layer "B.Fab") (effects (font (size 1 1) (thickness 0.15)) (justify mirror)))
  (pad "1" smd roundrect (at -1.0375 0 90) (size 1.175 1.45) (layers "B.Cu" "B.Paste" "B.Mask") (roundrect_rratio 0.212766) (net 4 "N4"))
  (pad "2" smd roundrect (at 1.0375 0 90) (size 1.175 1.45) (layers "B.Cu" "B.Paste" "B.Mask") (roundrect_rratio 0.212766) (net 2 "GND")))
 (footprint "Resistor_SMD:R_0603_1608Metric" (layer "B.Cu") (at 156.5 103.5 180)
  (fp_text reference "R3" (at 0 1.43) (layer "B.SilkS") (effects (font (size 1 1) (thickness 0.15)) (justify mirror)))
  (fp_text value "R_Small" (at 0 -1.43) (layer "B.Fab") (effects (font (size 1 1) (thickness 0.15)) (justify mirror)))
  (pad "1" smd roundrect (at -0.825 0 180) (size 0.8 0.95) (layers "B.Cu" "B.Paste" "B.Mask") (roundrect_rratio 0.25) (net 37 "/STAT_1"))
  (pad "2" smd roundrect (at 0.825 0 180) (size 0.8 0.95) (layers "B.Cu" "B.Paste" "B.Mask") (roundrect_rratio 0.25) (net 29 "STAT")))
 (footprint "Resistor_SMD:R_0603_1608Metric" (layer "B.Cu") (at 156.5 100.5 180)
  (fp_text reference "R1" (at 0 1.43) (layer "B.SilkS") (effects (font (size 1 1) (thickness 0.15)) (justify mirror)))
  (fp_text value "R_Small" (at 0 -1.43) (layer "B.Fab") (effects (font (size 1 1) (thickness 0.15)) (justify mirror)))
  (pad "1" smd roundrect (at -0.825 0 180) (size 0.8 0.95) (layers "B.Cu" "B.Paste" "B.Mask") (roundrect_rratio 0.25) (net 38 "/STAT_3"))
  (pad "2" smd roundrect (at 0.825 0 180) (size 0.8 0.95) (layers "B.Cu" "B.Paste" "B.Mask") (roundrect_rratio 0.25) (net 29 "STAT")))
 (gr_line (start 125 98.54) (end 125 105.54) (layer "Edge.Cuts") (width 0.1))
 (gr_line (start 157 96.54) (end 127 96.54) (layer "Edge.Cuts") (width 0.1))
 (gr_arc (start 125 98.54) (mid 125.585786 97.125786) (end 127 96.54) (layer "Edge.Cuts") (width 0.1))
 (gr_line (start 127 107.54) (end 157 107.54) (layer "Edge.Cuts") (width 0.1))
 (gr_arc (start 127 107.54) (mid 125.585786 106.954214) (end 125 105.54) (layer "Edge.Cuts") (width 0.1))
 (gr_arc (start 157 96.54) (mid 158.414214 97.125786) (end 159 98.54) (layer "Edge.Cuts") (width 0.1))
 (gr_line (start 159 98.54) (end 159 105.54) (layer "Edge.Cuts") (width 0.1))
 (gr_arc (start 159 105.54) (mid 158.414214 106.954214) (end 157 107.54) (layer "Edge.Cuts") (width 0.1))
 (segment (start 138.6175 98.12) (end 138.0375 97.54) (width 0.5) (layer "F.Cu") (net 1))
 (segment (start 140.525 98.12) (end 140.525 97.565) (width 0.5) (layer "F.Cu") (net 1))
 (segment (start 140.525 98.12) (end 140.525 97.515) (width 0.2) (layer "F.Cu") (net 1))
 (segment (start 139.1175 98.62) (end 138.0375 97.54) (width 0.3) (layer "F.Cu") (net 1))
 (segment (start 148.57 99.325) (end 148.57 100.5) (width 0.2) (layer "F.Cu") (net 1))
 (segment (start 140.525 98.12) (end 138.6175 98.12) (width 0.5) (layer "F.Cu") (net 1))
 (segment (start 140.525 98.62) (end 139.1175 98.62) (width 0.3) (layer "F.Cu") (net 1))
 (segment (start 140.525 97.565) (end 140 97.04) (width 0.5) (layer "F.Cu") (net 1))
 (segment (start 140.525 97.515) (end 141 97.04) (width 0.5) (layer "F.Cu") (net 1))
 (via (at 141 97.04) (size 0.8) (drill 0.4) (layers "F.Cu" "B.Cu") (free) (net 1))
 (via (at 140 97.04) (size 0.8) (drill 0.4) (layers "F.Cu" "B.Cu") (free) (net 1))
 (via (at 148.57 100.5) (size 0.8) (drill 0.4) (layers "F.Cu" "B.Cu") (free) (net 1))
 (segment (start 143.625 99.12) (end 142.075 99.12) (width 0.2) (layer "F.Cu") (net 2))
 (segment (start 143.625 98.62) (end 142.575 98.62) (width 0.2) (layer "F.Cu") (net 2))
 (segment (start 142.575 98.62) (end 142.075 99.12) (width 0.2) (layer "F.Cu") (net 2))
 (segment (start 145.5 99.365) (end 145.5 100.54) (width 0.2) (layer "F.Cu") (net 2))
 (via (at 145.5 100.54) (size 0.8) (drill 0.4) (layers "F.Cu" "B.Cu") (free) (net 2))
 (via (at 142 101.54) (size 0.8) (drill 0.4) (layers "F.Cu" "B.Cu") (free) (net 2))
 (segment (start 140.525 99.62) (end 140.525 99.12) (width 0.2) (layer "F.Cu") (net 3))
 (segment (start 140.525 99.12) (end 138.3825 99.12) (width 0.3) (layer "F.Cu") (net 3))
 (segment (start 146.5 98.5) (end 147 98) (width 0.2) (layer "F.Cu") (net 29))
 (segment (start 147.50452 96.99548) (end 152.99548 96.99548) (width 0.2) (layer "F.Cu") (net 29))
 (segment (start 152.99548 96.99548) (end 154 98) (width 0.2) (layer "F.Cu") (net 29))
 (segment (start 144.38 99.62) (end 144.5 99.5) (width 0.2) (layer "F.Cu") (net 29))
 (segment (start 143.625 99.62) (end 144.38 99.62) (width 0.2) (layer "F.Cu") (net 29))
 (segment (start 154 98) (end 154 100) (width 0.2) (layer "F.Cu") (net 29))
 (segment (start 147 97.5) (end 147.50452 96.99548) (width 0.2) (layer "F.Cu") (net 29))
 (segment (start 144.5 99.5) (end 144.5 99) (width 0.2) (layer "F.Cu") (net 29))
 (segment (start 147 97.7525) (end 147 97.5) (width 0.2) (layer "F.Cu") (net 29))
 (segment (start 147 98) (end 147 97.7525) (width 0.2) (layer "F.Cu") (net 29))
 (segment (start 154 100) (end 154.5 100.5) (width 0.2) (layer "F.Cu") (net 29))
 (segment (start 144.5 99) (end 145 98.5) (width 0.2) (layer "F.Cu") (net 29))
 (segment (start 145 98.5) (end 146.5 98.5) (width 0.2) (layer "F.Cu") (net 29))
 (via (at 154.5 100.5) (size 0.8) (drill 0.4) (layers "F.Cu" "B.Cu") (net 29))
 (segment (start 155.675 102) (end 155.675 103.5) (width 0.2) (layer "B.Cu") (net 29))
 (segment (start 155.675 100.5) (end 155.675 102) (width 0.2) (layer "B.Cu") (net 29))
 (segment (start 155.675 100.5) (end 154.5 100.5) (width 0.2) (layer "B.Cu") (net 29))
 (segment (start 157.21 102.29) (end 158.5 101) (width 0.2) (layer "F.Cu") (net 38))
 (segment (start 158.5 101) (end 158.5 100.5) (width 0.2) (layer "F.Cu") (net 38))
 (segment (start 152.2 102.29) (end 157.21 102.29) (width 0.2) (layer "F.Cu") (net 38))
 (via (at 158.5 100.5) (size 0.8) (drill 0.4) (layers "F.Cu" "B.Cu") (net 38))
 (segment (start 157.325 100.5) (end 158.5 100.5) (width 0.2) (layer "B.Cu") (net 38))
 (segment (start 152.2 102.79) (end 157.71 102.79) (width 0.2) (layer "F.Cu") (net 36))
 (segment (start 157.71 102.79) (end 158.5 102) (width 0.2) (layer "F.Cu") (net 36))
 (via (at 158.5 102) (size 0.8) (drill 0.4) (layers "F.Cu" "B.Cu") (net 36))
 (segment (start 157.325 102) (end 158.5 102) (width 0.2) (layer "B.Cu") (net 36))
 (segment (start 147 99.265) (end 148.57 97.695) (width 0.2) (layer "F.Cu") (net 5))
 (segment (start 147 99.3275) (end 147 99.265) (width 0.2) (layer "F.Cu") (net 5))
 (segment (start 152.2 103.29) (end 158.29 103.29) (width 0.2) (layer "F.Cu") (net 30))
 (segment (start 158.29 103.29) (end 158.5 103.5) (width 0.2) (layer "F.Cu") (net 30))
 (via (at 158.5 103.5) (size 0.8) (drill 0.4) (layers "F.Cu" "B.Cu") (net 30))
 (segment (start 157.325 103.5) (end 158.5 103.5) (width 0.2) (layer "B.Cu") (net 30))
 (segment (start 144.42 98.12) (end 143.625 98.12) (width 0.2) (layer "F.Cu") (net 6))
 (segment (start 145.5 97.715) (end 144.825 97.715) (width 0.2) (layer "F.Cu") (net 6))
 (segment (start 144.825 97.715) (end 144.42 98.12) (width 0.2) (layer "F.Cu") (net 6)))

